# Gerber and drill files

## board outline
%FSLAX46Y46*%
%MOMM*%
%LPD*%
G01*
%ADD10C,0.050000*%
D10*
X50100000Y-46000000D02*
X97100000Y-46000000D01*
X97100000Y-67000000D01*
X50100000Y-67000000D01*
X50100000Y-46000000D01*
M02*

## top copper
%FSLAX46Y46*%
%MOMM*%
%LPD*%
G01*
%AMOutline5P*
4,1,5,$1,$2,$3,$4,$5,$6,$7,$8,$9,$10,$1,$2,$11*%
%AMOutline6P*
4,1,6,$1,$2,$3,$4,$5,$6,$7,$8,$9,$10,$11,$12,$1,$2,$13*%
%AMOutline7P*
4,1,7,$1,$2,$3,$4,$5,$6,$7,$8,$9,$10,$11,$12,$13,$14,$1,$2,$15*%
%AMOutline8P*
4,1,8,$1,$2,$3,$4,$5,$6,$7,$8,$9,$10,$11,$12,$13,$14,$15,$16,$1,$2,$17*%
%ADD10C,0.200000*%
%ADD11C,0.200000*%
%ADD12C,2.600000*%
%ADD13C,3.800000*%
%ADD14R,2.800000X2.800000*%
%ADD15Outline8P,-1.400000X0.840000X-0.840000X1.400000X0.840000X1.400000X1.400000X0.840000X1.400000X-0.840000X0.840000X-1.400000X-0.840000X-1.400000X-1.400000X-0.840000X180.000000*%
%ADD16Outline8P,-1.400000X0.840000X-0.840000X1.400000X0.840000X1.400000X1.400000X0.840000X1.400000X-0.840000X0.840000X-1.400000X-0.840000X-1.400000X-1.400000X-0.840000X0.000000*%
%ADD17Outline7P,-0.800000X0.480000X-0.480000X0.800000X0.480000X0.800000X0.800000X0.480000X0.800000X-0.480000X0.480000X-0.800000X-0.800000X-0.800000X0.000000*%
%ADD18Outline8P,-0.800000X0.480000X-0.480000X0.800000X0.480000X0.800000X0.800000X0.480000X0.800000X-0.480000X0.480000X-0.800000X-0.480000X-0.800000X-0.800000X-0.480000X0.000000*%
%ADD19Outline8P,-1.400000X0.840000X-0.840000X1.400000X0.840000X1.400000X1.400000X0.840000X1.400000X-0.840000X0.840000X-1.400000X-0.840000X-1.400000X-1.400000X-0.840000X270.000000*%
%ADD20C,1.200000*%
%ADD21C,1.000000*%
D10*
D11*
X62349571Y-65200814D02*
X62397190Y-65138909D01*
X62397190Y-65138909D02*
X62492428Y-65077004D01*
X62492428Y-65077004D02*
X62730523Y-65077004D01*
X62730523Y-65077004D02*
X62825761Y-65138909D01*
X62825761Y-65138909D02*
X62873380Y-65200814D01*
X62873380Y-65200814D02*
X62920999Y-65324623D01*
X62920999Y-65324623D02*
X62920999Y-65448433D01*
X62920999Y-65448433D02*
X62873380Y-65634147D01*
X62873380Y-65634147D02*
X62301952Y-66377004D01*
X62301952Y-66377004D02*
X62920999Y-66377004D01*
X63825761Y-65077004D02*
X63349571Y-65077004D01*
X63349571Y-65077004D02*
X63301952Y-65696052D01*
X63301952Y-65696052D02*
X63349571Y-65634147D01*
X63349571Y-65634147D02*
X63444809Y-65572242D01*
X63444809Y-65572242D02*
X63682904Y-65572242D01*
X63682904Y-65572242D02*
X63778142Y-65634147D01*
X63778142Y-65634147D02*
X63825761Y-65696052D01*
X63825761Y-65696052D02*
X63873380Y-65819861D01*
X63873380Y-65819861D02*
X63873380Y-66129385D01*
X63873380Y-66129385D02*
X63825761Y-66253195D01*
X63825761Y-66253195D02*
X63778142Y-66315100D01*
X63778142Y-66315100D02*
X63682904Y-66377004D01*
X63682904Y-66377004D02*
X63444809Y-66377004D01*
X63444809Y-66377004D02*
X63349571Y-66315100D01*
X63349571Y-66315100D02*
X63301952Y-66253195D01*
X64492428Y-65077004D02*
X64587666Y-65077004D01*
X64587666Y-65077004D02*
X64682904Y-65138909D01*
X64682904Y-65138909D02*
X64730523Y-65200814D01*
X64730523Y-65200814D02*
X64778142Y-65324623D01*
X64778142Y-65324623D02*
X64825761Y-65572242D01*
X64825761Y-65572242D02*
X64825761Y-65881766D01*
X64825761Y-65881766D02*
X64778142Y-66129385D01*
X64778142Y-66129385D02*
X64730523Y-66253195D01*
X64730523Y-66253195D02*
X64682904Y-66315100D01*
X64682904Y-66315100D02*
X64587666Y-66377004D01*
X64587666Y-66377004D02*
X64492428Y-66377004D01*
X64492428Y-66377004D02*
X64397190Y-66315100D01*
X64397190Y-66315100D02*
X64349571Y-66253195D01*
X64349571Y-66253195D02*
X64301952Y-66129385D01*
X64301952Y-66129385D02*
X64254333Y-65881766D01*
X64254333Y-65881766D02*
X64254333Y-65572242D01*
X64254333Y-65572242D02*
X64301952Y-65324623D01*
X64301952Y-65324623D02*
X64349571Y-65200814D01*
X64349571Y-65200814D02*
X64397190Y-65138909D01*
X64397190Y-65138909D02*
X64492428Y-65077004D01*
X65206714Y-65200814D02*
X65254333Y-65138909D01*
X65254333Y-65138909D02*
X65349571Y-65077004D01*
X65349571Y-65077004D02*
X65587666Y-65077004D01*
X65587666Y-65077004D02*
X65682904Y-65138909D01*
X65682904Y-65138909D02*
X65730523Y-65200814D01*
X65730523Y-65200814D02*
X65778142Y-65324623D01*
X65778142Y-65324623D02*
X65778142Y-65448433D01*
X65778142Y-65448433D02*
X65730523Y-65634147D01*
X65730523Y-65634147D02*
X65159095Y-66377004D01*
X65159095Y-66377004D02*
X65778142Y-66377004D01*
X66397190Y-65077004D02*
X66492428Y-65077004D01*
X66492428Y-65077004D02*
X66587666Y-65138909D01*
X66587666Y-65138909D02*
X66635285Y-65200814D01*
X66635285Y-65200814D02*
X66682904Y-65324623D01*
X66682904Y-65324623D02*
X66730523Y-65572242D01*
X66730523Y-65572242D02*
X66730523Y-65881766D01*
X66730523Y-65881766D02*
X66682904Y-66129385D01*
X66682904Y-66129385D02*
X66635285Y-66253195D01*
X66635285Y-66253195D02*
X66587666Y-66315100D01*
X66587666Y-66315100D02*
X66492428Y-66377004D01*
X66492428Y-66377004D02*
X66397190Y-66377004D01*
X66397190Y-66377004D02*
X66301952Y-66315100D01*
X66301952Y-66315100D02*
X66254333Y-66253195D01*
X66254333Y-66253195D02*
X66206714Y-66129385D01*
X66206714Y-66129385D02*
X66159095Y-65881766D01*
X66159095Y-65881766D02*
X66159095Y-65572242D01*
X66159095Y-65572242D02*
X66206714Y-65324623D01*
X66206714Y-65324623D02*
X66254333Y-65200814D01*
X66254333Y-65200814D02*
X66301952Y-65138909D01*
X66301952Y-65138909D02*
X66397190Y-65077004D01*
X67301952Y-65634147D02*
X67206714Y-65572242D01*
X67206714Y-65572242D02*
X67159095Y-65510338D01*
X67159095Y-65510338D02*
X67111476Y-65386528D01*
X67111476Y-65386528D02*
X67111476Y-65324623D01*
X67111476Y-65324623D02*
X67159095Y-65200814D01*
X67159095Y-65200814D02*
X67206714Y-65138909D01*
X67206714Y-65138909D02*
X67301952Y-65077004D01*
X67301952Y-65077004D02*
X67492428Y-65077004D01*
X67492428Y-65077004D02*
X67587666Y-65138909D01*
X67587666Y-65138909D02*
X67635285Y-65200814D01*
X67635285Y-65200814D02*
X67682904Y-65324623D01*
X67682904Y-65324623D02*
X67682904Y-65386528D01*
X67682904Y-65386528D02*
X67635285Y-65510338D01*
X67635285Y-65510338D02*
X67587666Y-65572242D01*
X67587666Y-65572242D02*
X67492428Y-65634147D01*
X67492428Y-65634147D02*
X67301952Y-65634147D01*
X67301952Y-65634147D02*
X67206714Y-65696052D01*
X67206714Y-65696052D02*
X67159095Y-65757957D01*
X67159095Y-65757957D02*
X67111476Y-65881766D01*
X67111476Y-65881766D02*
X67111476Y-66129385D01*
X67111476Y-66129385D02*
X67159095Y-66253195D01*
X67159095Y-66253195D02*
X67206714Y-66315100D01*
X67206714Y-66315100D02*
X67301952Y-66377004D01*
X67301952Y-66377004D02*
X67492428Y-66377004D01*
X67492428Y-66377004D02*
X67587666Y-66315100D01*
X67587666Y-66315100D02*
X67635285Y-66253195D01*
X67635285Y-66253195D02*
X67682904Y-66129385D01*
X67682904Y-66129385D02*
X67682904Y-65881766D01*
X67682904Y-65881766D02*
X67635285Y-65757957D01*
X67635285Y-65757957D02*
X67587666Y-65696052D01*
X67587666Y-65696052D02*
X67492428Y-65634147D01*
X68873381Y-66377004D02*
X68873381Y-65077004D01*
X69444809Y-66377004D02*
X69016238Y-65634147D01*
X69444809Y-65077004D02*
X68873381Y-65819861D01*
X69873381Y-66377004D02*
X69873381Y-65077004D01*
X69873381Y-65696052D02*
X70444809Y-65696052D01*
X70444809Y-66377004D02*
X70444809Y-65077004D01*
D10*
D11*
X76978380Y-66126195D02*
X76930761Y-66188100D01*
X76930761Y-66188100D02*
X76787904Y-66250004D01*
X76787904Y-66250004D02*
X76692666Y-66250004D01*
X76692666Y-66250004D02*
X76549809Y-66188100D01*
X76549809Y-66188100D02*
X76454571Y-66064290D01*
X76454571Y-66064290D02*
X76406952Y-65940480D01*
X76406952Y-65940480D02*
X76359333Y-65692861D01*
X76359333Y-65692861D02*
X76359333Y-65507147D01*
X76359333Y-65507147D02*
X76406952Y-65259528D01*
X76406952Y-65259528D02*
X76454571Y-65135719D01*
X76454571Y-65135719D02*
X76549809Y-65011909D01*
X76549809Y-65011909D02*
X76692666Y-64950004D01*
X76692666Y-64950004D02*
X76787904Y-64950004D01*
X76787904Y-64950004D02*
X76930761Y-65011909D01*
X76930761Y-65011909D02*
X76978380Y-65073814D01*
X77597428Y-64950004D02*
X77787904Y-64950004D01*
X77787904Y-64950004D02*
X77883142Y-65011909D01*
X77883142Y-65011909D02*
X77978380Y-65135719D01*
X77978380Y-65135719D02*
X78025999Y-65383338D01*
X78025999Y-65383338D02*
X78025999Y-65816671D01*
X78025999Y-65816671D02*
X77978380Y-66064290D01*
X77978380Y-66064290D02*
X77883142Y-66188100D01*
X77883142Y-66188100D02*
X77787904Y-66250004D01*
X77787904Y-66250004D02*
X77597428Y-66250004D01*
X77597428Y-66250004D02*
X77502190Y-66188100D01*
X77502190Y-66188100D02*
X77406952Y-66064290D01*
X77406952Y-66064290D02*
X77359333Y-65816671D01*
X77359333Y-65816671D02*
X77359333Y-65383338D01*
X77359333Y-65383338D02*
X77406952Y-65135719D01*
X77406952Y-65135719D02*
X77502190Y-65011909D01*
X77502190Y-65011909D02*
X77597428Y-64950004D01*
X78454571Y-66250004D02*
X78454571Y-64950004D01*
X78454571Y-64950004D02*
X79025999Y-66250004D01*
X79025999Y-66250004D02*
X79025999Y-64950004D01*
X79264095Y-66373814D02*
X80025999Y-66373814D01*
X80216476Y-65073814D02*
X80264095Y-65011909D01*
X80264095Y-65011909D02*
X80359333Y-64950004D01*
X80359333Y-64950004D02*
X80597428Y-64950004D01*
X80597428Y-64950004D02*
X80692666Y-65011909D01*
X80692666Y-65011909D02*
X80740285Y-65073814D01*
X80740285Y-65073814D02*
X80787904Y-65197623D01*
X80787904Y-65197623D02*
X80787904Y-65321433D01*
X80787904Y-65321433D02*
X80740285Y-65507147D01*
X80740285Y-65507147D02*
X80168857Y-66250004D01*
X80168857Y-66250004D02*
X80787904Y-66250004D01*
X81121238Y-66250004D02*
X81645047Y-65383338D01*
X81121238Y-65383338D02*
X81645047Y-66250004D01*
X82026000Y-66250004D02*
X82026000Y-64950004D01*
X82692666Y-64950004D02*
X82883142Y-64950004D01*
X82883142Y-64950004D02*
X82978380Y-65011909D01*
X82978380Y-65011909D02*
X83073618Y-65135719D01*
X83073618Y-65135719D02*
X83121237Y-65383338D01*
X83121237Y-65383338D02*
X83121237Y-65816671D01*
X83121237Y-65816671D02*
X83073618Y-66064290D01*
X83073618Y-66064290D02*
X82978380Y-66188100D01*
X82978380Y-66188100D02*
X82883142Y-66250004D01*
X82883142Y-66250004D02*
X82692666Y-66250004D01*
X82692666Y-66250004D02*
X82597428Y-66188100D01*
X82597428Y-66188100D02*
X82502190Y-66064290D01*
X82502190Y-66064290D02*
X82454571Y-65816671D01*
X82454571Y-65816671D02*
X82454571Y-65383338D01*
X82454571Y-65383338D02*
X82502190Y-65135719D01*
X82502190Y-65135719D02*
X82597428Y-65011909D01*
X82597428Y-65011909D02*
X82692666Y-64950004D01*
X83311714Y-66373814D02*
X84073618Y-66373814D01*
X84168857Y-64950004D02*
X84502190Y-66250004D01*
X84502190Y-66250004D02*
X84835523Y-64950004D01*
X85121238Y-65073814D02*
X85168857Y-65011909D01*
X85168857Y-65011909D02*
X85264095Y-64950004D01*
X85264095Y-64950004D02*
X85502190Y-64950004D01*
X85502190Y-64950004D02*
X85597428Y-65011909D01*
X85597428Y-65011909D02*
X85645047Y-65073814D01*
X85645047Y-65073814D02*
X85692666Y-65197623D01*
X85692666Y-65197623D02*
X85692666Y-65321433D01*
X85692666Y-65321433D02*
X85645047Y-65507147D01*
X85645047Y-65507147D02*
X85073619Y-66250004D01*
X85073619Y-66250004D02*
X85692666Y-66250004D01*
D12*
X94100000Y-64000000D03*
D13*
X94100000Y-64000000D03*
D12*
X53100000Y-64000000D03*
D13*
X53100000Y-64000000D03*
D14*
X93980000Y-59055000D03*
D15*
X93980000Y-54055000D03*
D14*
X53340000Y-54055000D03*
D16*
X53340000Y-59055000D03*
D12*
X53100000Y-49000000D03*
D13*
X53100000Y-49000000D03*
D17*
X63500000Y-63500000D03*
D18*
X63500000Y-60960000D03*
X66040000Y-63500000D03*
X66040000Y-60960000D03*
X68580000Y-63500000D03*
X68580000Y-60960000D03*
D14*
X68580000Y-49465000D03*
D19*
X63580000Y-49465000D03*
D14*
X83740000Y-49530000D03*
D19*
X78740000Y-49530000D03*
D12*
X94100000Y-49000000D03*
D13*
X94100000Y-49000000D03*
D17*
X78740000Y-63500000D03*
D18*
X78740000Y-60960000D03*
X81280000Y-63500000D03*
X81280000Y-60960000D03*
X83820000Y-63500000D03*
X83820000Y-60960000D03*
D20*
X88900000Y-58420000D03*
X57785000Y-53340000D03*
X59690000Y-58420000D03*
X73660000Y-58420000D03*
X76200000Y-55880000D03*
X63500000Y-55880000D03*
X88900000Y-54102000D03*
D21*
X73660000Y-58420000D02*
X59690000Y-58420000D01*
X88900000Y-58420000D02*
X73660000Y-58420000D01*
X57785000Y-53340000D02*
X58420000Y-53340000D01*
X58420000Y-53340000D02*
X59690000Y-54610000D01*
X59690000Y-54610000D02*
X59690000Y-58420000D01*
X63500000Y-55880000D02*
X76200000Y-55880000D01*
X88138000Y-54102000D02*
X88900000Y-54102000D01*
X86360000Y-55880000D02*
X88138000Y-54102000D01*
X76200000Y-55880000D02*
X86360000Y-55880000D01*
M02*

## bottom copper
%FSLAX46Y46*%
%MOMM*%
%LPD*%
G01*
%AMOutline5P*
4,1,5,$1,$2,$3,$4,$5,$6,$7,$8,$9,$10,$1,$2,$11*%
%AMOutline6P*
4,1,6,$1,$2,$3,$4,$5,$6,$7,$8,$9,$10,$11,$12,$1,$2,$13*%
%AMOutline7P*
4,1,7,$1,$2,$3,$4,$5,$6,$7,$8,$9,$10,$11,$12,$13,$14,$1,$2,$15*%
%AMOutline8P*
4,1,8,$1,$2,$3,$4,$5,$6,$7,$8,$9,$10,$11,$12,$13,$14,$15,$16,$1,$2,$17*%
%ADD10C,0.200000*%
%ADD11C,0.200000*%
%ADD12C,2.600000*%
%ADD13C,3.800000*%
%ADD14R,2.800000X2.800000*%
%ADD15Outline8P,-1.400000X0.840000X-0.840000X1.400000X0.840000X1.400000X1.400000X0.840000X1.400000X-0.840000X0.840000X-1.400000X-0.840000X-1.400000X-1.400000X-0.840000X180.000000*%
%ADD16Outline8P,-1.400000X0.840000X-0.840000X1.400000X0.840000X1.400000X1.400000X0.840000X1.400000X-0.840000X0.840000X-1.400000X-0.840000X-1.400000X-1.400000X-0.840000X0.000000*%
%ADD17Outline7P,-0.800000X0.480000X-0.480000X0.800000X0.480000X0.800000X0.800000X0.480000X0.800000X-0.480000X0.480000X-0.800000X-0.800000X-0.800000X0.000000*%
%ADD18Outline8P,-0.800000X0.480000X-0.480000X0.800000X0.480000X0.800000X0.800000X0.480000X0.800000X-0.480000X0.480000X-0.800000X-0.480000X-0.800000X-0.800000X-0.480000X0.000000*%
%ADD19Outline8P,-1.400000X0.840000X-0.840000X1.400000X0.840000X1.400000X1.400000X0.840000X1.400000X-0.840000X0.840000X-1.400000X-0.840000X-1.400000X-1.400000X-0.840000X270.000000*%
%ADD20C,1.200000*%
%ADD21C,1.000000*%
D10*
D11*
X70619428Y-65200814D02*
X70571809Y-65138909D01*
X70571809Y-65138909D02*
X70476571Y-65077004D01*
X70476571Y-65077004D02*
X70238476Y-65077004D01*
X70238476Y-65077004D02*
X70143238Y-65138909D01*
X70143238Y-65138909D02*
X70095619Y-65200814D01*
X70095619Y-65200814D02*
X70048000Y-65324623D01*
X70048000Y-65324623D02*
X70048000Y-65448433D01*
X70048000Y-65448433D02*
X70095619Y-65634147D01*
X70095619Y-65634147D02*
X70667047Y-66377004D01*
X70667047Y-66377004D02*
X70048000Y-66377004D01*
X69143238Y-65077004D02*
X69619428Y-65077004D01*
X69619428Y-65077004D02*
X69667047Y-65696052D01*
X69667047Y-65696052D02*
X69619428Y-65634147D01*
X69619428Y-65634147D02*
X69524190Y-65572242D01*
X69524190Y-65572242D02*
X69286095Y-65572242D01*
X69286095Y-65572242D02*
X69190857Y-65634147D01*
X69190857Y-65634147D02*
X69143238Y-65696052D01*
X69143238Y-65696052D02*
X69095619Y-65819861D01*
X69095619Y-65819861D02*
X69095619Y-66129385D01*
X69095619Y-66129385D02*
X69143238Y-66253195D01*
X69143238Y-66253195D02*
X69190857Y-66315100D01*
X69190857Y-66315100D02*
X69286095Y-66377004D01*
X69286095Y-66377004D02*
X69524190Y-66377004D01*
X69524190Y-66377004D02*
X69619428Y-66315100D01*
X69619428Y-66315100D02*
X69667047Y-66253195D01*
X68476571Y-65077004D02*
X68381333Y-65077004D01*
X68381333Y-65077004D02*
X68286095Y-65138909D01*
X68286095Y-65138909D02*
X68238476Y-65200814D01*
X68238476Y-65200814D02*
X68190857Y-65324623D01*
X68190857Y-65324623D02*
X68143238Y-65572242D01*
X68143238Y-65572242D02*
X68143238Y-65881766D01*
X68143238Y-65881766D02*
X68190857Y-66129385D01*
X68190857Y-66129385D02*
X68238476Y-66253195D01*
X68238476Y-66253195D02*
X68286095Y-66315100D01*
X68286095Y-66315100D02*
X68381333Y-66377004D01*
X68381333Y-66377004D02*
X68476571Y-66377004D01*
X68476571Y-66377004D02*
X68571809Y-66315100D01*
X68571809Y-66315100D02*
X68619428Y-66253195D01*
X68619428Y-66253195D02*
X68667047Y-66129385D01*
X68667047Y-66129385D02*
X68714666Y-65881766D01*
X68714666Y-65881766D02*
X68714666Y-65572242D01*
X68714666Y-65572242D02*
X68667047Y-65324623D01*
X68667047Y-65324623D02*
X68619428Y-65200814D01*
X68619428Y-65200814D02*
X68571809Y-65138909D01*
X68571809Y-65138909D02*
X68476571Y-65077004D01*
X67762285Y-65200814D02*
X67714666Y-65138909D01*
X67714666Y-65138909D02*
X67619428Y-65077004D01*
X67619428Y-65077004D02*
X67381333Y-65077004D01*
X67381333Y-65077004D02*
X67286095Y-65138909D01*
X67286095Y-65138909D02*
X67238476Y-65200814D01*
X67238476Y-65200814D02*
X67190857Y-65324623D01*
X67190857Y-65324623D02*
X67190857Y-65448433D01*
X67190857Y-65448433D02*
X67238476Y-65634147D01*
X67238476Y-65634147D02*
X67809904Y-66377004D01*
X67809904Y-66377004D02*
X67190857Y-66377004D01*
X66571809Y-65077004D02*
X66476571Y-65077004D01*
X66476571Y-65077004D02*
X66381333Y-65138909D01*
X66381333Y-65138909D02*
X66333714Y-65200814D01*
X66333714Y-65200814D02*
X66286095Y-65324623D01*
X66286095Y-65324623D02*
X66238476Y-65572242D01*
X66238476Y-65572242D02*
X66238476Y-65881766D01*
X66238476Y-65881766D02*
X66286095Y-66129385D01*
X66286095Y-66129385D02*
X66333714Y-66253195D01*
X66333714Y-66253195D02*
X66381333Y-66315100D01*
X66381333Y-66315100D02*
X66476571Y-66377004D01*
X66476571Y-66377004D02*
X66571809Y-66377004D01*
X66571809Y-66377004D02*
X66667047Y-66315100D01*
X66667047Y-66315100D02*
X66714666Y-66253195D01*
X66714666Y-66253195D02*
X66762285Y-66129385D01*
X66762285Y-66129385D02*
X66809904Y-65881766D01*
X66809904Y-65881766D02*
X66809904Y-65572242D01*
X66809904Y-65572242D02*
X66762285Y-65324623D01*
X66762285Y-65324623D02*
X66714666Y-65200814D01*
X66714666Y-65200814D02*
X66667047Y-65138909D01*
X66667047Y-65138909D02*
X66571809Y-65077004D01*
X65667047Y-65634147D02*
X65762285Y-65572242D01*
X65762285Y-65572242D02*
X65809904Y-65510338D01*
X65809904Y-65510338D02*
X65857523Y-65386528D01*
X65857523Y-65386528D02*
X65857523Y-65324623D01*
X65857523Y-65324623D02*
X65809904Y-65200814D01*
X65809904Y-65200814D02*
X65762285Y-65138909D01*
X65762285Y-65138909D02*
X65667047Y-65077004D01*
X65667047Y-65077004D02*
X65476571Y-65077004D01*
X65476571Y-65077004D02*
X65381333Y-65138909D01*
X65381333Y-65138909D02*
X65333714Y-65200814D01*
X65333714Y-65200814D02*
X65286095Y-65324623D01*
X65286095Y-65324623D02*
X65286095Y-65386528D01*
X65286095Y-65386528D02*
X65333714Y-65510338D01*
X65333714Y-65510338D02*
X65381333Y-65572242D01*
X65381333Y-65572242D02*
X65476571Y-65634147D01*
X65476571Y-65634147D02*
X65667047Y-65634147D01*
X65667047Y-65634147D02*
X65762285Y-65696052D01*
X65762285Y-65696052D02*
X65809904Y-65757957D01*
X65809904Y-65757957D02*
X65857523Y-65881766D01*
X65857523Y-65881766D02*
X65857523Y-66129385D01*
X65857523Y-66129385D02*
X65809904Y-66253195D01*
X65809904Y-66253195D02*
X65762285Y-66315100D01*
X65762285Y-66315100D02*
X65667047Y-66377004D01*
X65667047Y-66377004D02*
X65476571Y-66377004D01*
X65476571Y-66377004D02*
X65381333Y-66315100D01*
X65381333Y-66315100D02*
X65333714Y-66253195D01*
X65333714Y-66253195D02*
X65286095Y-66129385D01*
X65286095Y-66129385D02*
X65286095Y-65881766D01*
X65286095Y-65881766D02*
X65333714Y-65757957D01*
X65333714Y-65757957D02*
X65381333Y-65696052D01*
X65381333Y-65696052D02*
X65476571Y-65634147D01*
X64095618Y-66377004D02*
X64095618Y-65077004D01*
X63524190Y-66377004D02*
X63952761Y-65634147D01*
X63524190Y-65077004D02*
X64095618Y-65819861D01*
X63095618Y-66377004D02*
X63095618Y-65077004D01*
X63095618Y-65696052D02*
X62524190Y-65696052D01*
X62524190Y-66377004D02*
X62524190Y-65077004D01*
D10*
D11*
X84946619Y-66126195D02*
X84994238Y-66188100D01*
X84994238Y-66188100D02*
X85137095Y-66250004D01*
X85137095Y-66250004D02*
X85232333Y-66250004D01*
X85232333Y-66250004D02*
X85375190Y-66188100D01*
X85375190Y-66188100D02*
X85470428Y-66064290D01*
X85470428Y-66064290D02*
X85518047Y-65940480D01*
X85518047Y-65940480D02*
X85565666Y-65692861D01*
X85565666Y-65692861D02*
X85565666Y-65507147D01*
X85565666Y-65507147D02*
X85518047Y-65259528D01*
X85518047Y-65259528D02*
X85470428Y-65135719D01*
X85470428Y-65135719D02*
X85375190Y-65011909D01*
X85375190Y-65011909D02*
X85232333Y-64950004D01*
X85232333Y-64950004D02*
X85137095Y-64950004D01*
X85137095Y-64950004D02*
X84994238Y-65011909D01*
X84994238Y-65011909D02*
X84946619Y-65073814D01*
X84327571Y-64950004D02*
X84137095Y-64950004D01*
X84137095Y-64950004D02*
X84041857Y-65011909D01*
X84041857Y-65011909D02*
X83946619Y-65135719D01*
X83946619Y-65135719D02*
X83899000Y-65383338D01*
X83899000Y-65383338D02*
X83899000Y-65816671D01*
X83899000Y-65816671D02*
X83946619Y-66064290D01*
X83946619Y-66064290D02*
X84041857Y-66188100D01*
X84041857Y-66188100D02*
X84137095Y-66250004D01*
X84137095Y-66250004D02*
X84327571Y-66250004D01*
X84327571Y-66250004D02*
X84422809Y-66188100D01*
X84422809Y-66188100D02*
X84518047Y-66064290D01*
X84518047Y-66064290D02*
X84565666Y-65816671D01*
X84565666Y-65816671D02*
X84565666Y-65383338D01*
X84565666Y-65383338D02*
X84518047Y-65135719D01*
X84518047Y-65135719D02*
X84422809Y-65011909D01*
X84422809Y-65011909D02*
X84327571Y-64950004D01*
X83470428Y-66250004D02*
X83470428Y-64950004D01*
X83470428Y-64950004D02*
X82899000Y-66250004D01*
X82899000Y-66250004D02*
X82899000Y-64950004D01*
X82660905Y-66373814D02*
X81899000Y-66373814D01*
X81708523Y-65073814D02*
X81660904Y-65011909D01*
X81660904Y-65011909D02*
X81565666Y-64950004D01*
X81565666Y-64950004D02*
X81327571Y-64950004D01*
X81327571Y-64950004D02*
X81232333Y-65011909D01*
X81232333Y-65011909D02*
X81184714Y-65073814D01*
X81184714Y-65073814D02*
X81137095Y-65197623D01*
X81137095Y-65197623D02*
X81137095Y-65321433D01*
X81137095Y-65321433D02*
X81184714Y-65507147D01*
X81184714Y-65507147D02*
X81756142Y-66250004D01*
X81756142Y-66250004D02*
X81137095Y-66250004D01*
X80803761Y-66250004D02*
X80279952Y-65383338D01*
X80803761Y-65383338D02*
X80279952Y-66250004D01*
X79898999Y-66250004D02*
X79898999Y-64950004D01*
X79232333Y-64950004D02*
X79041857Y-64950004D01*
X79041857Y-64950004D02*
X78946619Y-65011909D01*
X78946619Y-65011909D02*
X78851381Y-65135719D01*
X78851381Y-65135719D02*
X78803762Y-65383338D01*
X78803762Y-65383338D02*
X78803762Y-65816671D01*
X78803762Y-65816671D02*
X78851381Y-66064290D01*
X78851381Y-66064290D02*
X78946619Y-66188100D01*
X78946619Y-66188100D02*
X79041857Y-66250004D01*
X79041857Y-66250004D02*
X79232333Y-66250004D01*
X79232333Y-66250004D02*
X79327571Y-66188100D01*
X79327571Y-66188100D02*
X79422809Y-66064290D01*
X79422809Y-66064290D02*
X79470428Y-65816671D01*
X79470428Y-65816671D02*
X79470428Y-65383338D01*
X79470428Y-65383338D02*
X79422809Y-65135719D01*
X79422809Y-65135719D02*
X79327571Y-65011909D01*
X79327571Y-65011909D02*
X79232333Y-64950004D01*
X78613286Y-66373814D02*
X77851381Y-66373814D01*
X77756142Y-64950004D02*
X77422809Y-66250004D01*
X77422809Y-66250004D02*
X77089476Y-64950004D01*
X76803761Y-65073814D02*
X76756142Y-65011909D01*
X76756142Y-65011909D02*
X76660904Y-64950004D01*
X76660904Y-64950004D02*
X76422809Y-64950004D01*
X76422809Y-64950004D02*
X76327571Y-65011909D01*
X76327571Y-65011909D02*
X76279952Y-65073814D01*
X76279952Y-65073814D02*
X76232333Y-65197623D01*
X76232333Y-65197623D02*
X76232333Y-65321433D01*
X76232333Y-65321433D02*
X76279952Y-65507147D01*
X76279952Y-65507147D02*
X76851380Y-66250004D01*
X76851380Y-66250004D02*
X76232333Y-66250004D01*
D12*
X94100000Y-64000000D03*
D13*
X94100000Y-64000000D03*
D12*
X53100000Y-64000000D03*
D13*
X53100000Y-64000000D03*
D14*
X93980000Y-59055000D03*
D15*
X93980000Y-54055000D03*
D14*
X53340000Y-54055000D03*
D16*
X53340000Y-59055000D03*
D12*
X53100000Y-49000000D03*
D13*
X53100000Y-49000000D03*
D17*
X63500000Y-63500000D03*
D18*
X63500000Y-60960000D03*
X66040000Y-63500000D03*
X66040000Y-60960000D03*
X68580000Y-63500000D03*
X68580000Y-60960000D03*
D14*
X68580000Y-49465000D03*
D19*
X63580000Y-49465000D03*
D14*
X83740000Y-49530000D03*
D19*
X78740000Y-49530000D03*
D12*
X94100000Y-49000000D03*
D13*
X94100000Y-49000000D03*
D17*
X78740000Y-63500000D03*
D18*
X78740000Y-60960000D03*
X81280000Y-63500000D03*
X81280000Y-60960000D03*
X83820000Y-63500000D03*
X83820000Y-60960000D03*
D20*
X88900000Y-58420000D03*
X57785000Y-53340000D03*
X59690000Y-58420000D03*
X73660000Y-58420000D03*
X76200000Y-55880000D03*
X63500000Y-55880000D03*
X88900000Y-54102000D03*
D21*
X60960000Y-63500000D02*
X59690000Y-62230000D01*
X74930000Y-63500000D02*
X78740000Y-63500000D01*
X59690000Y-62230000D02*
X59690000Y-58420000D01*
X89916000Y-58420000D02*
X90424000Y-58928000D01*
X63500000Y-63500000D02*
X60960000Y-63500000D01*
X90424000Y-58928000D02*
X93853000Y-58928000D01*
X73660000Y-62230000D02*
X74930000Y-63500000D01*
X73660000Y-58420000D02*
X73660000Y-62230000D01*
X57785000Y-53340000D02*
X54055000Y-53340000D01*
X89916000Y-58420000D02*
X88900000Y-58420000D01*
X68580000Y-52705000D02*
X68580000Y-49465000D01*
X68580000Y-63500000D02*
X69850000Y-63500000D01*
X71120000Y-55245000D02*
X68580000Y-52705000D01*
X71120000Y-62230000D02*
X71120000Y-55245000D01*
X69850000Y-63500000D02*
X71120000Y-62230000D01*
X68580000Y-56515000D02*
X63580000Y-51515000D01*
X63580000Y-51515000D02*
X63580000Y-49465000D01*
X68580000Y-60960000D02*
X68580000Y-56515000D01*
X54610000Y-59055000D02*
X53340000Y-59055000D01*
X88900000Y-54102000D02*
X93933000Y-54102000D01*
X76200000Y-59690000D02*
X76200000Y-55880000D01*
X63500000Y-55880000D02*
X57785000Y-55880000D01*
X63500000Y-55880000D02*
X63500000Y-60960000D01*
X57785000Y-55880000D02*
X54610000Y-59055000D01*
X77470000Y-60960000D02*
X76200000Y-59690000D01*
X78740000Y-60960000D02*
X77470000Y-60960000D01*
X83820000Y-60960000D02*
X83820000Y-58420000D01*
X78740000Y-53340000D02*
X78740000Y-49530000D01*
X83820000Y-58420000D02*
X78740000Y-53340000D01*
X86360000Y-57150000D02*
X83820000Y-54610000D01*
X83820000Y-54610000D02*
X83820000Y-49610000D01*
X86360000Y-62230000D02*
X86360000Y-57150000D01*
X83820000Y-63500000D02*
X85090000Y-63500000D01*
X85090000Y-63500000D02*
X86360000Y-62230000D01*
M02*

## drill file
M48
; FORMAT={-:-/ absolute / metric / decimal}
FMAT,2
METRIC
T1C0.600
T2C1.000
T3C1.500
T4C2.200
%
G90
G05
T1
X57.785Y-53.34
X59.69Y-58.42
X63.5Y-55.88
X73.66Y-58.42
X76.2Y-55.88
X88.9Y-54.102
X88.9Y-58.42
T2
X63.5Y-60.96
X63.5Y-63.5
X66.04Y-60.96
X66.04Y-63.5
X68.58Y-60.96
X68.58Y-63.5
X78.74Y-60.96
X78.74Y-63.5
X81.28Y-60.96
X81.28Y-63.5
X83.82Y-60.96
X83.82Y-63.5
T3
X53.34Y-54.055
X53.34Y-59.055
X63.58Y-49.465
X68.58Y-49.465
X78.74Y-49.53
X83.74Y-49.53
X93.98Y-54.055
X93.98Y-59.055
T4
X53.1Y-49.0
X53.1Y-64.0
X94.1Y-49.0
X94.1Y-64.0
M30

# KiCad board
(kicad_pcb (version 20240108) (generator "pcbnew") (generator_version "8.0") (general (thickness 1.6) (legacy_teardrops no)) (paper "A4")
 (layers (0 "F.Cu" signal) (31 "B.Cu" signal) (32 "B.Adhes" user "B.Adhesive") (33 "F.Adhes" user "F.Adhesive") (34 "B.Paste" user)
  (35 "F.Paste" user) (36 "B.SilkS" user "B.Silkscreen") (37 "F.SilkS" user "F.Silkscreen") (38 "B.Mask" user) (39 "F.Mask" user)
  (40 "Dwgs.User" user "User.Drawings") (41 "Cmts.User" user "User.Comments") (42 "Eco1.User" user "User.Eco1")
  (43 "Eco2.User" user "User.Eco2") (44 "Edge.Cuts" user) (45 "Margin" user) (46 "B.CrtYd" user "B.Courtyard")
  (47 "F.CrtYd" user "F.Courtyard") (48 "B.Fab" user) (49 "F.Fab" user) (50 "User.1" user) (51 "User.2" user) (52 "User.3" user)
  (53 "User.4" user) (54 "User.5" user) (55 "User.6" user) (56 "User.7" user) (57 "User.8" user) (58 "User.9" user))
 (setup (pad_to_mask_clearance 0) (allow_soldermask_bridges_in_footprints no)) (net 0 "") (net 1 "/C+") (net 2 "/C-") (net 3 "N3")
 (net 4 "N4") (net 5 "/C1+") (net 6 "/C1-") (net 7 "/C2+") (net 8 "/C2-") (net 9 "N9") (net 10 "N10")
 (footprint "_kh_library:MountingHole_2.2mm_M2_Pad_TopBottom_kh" (layer "F.Cu") (at 94.1 64)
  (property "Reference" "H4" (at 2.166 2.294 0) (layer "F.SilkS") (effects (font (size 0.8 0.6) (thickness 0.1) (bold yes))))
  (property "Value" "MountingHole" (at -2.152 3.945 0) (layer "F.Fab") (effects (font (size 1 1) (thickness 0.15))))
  (pad "1" thru_hole circle (at 0 0) (size 2.6 2.6) (drill 2.2) (layers "*.Cu" "*.Mask") (remove_unused_layers no))
  (pad "1" connect circle (at 0 0) (size 3.8 3.8) (layers "F.Cu" "F.Mask"))
  (pad "1" connect circle (at 0 0) (size 3.8 3.8) (layers "B.Cu" "B.Mask")))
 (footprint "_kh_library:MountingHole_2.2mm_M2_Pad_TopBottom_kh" (layer "F.Cu") (at 53.1 64)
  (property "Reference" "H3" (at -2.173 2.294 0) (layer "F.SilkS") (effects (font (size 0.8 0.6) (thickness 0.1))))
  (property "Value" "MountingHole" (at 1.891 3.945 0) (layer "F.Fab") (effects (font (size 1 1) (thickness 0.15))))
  (pad "1" thru_hole circle (at 0 0) (size 2.6 2.6) (drill 2.2) (layers "*.Cu" "*.Mask") (remove_unused_layers no))
  (pad "1" connect circle (at 0 0) (size 3.8 3.8) (layers "F.Cu" "F.Mask"))
  (pad "1" connect circle (at 0 0) (size 3.8 3.8) (layers "B.Cu" "B.Mask")))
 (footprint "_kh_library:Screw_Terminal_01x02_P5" (layer "F.Cu") (at 93.98 59.055 180)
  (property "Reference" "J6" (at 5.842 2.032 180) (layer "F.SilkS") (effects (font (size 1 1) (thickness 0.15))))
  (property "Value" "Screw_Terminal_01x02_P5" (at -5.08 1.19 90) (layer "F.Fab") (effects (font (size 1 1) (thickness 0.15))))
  (pad "1" thru_hole rect (at 0 0 180) (size 2.8 2.8) (drill 1.5) (layers "*.Cu" "*.Mask") (remove_unused_layers no) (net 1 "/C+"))
  (pad "2" thru_hole roundrect (at 0 5 180) (size 2.8 2.8) (drill 1.5) (layers "*.Cu" "*.Mask") (remove_unused_layers no)
   (roundrect_rratio 0) (chamfer_ratio 0.2) (chamfer top_left top_right bottom_left bottom_right) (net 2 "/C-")))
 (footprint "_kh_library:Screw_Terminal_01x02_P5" (layer "F.Cu") (at 53.34 54.055)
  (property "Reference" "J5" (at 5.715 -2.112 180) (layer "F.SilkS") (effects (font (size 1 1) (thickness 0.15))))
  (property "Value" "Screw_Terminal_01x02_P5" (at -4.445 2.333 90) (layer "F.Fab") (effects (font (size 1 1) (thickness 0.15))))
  (pad "1" thru_hole rect (at 0 0) (size 2.8 2.8) (drill 1.5) (layers "*.Cu" "*.Mask") (remove_unused_layers no) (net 1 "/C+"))
  (pad "2" thru_hole roundrect (at 0 5) (size 2.8 2.8) (drill 1.5) (layers "*.Cu" "*.Mask") (remove_unused_layers no) (roundrect_rratio 0)
   (chamfer_ratio 0.2) (chamfer top_left top_right bottom_left bottom_right) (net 2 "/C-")))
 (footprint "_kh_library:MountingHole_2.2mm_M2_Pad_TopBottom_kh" (layer "F.Cu") (at 53.1 49)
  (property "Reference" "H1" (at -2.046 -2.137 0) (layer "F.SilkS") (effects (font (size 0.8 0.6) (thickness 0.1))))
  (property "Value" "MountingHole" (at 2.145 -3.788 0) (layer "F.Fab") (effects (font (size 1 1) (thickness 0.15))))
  (pad "1" thru_hole circle (at 0 0) (size 2.6 2.6) (drill 2.2) (layers "*.Cu" "*.Mask") (remove_unused_layers no))
  (pad "1" connect circle (at 0 0) (size 3.8 3.8) (layers "F.Cu" "F.Mask"))
  (pad "1" connect circle (at 0 0) (size 3.8 3.8) (layers "B.Cu" "B.Mask")))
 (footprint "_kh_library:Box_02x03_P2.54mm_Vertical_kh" (layer "F.Cu") (at 63.5 63.5)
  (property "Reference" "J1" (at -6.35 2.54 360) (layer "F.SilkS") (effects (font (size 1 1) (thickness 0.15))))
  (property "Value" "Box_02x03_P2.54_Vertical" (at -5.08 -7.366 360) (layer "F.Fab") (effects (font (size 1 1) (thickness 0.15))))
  (pad "1" thru_hole roundrect (at 0 0) (size 1.6 1.6) (drill 1) (layers "*.Cu" "*.Mask") (remove_unused_layers no) (roundrect_rratio 0)
   (chamfer_ratio 0.2) (chamfer top_left top_right bottom_right) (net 1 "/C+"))
  (pad "2" thru_hole roundrect (at 0 -2.54) (size 1.6 1.6) (drill 1) (layers "*.Cu" "*.Mask") (remove_unused_layers no) (roundrect_rratio 0)
   (chamfer_ratio 0.2) (chamfer top_left top_right bottom_left bottom_right) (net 2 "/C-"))
  (pad "3" thru_hole roundrect (at 2.54 0) (size 1.6 1.6) (drill 1) (layers "*.Cu" "*.Mask") (remove_unused_layers no) (roundrect_rratio 0)
   (chamfer_ratio 0.2) (chamfer top_left top_right bottom_left bottom_right) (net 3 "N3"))
  (pad "4" thru_hole roundrect (at 2.54 -2.54) (size 1.6 1.6) (drill 1) (layers "*.Cu" "*.Mask") (remove_unused_layers no)
   (roundrect_rratio 0) (chamfer_ratio 0.2) (chamfer top_left top_right bottom_left bottom_right) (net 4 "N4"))
  (pad "5" thru_hole roundrect (at 5.08 0) (size 1.6 1.6) (drill 1) (layers "*.Cu" "*.Mask") (remove_unused_layers no) (roundrect_rratio 0)
   (chamfer_ratio 0.2) (chamfer top_left top_right bottom_left bottom_right) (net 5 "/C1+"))
  (pad "6" thru_hole roundrect (at 5.08 -2.54) (size 1.6 1.6) (drill 1) (layers "*.Cu" "*.Mask") (remove_unused_layers no)
   (roundrect_rratio 0) (chamfer_ratio 0.2) (chamfer top_left top_right bottom_left bottom_right) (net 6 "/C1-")))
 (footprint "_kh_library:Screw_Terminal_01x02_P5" (layer "F.Cu") (at 68.58 49.465 -90)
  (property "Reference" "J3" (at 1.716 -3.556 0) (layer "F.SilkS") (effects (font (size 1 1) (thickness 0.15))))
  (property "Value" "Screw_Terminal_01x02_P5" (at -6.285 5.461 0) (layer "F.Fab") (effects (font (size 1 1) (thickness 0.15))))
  (pad "1" thru_hole rect (at 0 0 270) (size 2.8 2.8) (drill 1.5) (layers "*.Cu" "*.Mask") (remove_unused_layers no) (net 5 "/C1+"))
  (pad "2" thru_hole roundrect (at 0 5 270) (size 2.8 2.8) (drill 1.5) (layers "*.Cu" "*.Mask") (remove_unused_layers no)
   (roundrect_rratio 0) (chamfer_ratio 0.2) (chamfer top_left top_right bottom_left bottom_right) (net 6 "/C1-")))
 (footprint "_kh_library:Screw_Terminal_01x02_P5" (layer "F.Cu") (at 83.74 49.53 -90)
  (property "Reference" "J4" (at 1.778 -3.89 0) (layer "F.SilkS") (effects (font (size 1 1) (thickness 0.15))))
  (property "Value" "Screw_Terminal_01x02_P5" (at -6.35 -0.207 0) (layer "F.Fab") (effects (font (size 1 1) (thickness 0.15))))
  (pad "1" thru_hole rect (at 0 0 270) (size 2.8 2.8) (drill 1.5) (layers "*.Cu" "*.Mask") (remove_unused_layers no) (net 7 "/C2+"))
  (pad "2" thru_hole roundrect (at 0 5 270) (size 2.8 2.8) (drill 1.5) (layers "*.Cu" "*.Mask") (remove_unused_layers no)
   (roundrect_rratio 0) (chamfer_ratio 0.2) (chamfer top_left top_right bottom_left bottom_right) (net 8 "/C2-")))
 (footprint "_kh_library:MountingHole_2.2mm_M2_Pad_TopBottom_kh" (layer "F.Cu") (at 94.1 49)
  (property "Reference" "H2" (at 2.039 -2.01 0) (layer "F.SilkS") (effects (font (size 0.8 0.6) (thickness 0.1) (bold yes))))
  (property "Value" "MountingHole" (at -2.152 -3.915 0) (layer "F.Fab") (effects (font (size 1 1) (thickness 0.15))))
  (pad "1" thru_hole circle (at 0 0) (size 2.6 2.6) (drill 2.2) (layers "*.Cu" "*.Mask") (remove_unused_layers no))
  (pad "1" connect circle (at 0 0) (size 3.8 3.8) (layers "F.Cu" "F.Mask"))
  (pad "1" connect circle (at 0 0) (size 3.8 3.8) (layers "B.Cu" "B.Mask")))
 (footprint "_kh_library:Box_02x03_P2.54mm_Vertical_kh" (layer "F.Cu") (at 78.74 63.5)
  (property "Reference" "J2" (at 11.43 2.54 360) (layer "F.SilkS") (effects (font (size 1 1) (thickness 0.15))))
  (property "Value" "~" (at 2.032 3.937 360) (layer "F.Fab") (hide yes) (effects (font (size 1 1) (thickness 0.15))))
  (pad "1" thru_hole roundrect (at 0 0) (size 1.6 1.6) (drill 1) (layers "*.Cu" "*.Mask") (remove_unused_layers no) (roundrect_rratio 0)
   (chamfer_ratio 0.2) (chamfer top_left top_right bottom_right) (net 1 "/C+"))
  (pad "2" thru_hole roundrect (at 0 -2.54) (size 1.6 1.6) (drill 1) (layers "*.Cu" "*.Mask") (remove_unused_layers no) (roundrect_rratio 0)
   (chamfer_ratio 0.2) (chamfer top_left top_right bottom_left bottom_right) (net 2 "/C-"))
  (pad "3" thru_hole roundrect (at 2.54 0) (size 1.6 1.6) (drill 1) (layers "*.Cu" "*.Mask") (remove_unused_layers no) (roundrect_rratio 0)
   (chamfer_ratio 0.2) (chamfer top_left top_right bottom_left bottom_right) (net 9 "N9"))
  (pad "4" thru_hole roundrect (at 2.54 -2.54) (size 1.6 1.6) (drill 1) (layers "*.Cu" "*.Mask") (remove_unused_layers no)
   (roundrect_rratio 0) (chamfer_ratio 0.2) (chamfer top_left top_right bottom_left bottom_right) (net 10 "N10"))
  (pad "5" thru_hole roundrect (at 5.08 0) (size 1.6 1.6) (drill 1) (layers "*.Cu" "*.Mask") (remove_unused_layers no) (roundrect_rratio 0)
   (chamfer_ratio 0.2) (chamfer top_left top_right bottom_left bottom_right) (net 7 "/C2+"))
  (pad "6" thru_hole roundrect (at 5.08 -2.54) (size 1.6 1.6) (drill 1) (layers "*.Cu" "*.Mask") (remove_unused_layers no)
   (roundrect_rratio 0) (chamfer_ratio 0.2) (chamfer top_left top_right bottom_left bottom_right) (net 8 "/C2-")))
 (gr_rect (start 50.1 46) (end 97.1 67) (stroke (width 0.05) (type default)) (fill none) (layer "Edge.Cuts"))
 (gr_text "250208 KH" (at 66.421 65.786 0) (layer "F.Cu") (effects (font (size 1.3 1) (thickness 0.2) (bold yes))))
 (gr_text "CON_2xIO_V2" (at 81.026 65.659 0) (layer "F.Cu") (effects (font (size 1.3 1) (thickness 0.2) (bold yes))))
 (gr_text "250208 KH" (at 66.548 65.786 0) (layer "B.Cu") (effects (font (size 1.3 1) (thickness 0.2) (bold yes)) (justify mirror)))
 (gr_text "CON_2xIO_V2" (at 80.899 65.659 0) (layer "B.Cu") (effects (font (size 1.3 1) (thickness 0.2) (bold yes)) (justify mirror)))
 (segment (start 73.66 58.42) (end 59.69 58.42) (width 1) (layer "F.Cu") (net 1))
 (segment (start 88.9 58.42) (end 73.66 58.42) (width 1) (layer "F.Cu") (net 1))
 (segment (start 57.785 53.34) (end 58.42 53.34) (width 1) (layer "F.Cu") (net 1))
 (segment (start 58.42 53.34) (end 59.69 54.61) (width 1) (layer "F.Cu") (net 1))
 (segment (start 59.69 54.61) (end 59.69 58.42) (width 1) (layer "F.Cu") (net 1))
 (via (at 88.9 58.42) (size 1.2) (drill 0.6) (layers "F.Cu" "B.Cu") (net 1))
 (via (at 57.785 53.34) (size 1.2) (drill 0.6) (layers "F.Cu" "B.Cu") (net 1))
 (via (at 59.69 58.42) (size 1.2) (drill 0.6) (layers "F.Cu" "B.Cu") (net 1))
 (via (at 73.66 58.42) (size 1.2) (drill 0.6) (layers "F.Cu" "B.Cu") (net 1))
 (segment (start 60.96 63.5) (end 59.69 62.23) (width 1) (layer "B.Cu") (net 1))
 (segment (start 74.93 63.5) (end 78.74 63.5) (width 1) (layer "B.Cu") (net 1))
 (segment (start 59.69 62.23) (end 59.69 58.42) (width 1) (layer "B.Cu") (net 1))
 (segment (start 89.916 58.42) (end 90.424 58.928) (width 1) (layer "B.Cu") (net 1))
 (segment (start 63.5 63.5) (end 60.96 63.5) (width 1) (layer "B.Cu") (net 1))
 (segment (start 90.424 58.928) (end 93.853 58.928) (width 1) (layer "B.Cu") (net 1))
 (segment (start 73.66 62.23) (end 74.93 63.5) (width 1) (layer "B.Cu") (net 1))
 (segment (start 73.66 58.42) (end 73.66 62.23) (width 1) (layer "B.Cu") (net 1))
 (segment (start 57.785 53.34) (end 54.055 53.34) (width 1) (layer "B.Cu") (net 1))
 (segment (start 89.916 58.42) (end 88.9 58.42) (width 1) (layer "B.Cu") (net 1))
 (segment (start 68.58 52.705) (end 68.58 49.465) (width 1) (layer "B.Cu") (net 5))
 (segment (start 68.58 63.5) (end 69.85 63.5) (width 1) (layer "B.Cu") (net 5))
 (segment (start 71.12 55.245) (end 68.58 52.705) (width 1) (layer "B.Cu") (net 5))
 (segment (start 71.12 62.23) (end 71.12 55.245) (width 1) (layer "B.Cu") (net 5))
 (segment (start 69.85 63.5) (end 71.12 62.23) (width 1) (layer "B.Cu") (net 5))
 (segment (start 68.58 56.515) (end 63.58 51.515) (width 1) (layer "B.Cu") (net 6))
 (segment (start 63.58 51.515) (end 63.58 49.465) (width 1) (layer "B.Cu") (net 6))
 (segment (start 68.58 60.96) (end 68.58 56.515) (width 1) (layer "B.Cu") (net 6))
 (segment (start 63.5 55.88) (end 76.2 55.88) (width 1) (layer "F.Cu") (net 2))
 (segment (start 88.138 54.102) (end 88.9 54.102) (width 1) (layer "F.Cu") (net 2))
 (segment (start 86.36 55.88) (end 88.138 54.102) (width 1) (layer "F.Cu") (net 2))
 (segment (start 76.2 55.88) (end 86.36 55.88) (width 1) (layer "F.Cu") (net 2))
 (via (at 76.2 55.88) (size 1.2) (drill 0.6) (layers "F.Cu" "B.Cu") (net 2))
 (via (at 63.5 55.88) (size 1.2) (drill 0.6) (layers "F.Cu" "B.Cu") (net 2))
 (via (at 88.9 54.102) (size 1.2) (drill 0.6) (layers "F.Cu" "B.Cu") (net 2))
 (segment (start 54.61 59.055) (end 53.34 59.055) (width 1) (layer "B.Cu") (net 2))
 (segment (start 88.9 54.102) (end 93.933 54.102) (width 1) (layer "B.Cu") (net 2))
 (segment (start 76.2 59.69) (end 76.2 55.88) (width 1) (layer "B.Cu") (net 2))
 (segment (start 63.5 55.88) (end 57.785 55.88) (width 1) (layer "B.Cu") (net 2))
 (segment (start 63.5 55.88) (end 63.5 60.96) (width 1) (layer "B.Cu") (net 2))
 (segment (start 57.785 55.88) (end 54.61 59.055) (width 1) (layer "B.Cu") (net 2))
 (segment (start 77.47 60.96) (end 76.2 59.69) (width 1) (layer "B.Cu") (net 2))
 (segment (start 78.74 60.96) (end 77.47 60.96) (width 1) (layer "B.Cu") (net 2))
 (segment (start 83.82 60.96) (end 83.82 58.42) (width 1) (layer "B.Cu") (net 8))
 (segment (start 78.74 53.34) (end 78.74 49.53) (width 1) (layer "B.Cu") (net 8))
 (segment (start 83.82 58.42) (end 78.74 53.34) (width 1) (layer "B.Cu") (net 8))
 (segment (start 86.36 57.15) (end 83.82 54.61) (width 1) (layer "B.Cu") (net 7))
 (segment (start 83.82 54.61) (end 83.82 49.61) (width 1) (layer "B.Cu") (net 7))
 (segment (start 86.36 62.23) (end 86.36 57.15) (width 1) (layer "B.Cu") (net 7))
 (segment (start 83.82 63.5) (end 85.09 63.5) (width 1) (layer "B.Cu") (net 7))
 (segment (start 85.09 63.5) (end 86.36 62.23) (width 1) (layer "B.Cu") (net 7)))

